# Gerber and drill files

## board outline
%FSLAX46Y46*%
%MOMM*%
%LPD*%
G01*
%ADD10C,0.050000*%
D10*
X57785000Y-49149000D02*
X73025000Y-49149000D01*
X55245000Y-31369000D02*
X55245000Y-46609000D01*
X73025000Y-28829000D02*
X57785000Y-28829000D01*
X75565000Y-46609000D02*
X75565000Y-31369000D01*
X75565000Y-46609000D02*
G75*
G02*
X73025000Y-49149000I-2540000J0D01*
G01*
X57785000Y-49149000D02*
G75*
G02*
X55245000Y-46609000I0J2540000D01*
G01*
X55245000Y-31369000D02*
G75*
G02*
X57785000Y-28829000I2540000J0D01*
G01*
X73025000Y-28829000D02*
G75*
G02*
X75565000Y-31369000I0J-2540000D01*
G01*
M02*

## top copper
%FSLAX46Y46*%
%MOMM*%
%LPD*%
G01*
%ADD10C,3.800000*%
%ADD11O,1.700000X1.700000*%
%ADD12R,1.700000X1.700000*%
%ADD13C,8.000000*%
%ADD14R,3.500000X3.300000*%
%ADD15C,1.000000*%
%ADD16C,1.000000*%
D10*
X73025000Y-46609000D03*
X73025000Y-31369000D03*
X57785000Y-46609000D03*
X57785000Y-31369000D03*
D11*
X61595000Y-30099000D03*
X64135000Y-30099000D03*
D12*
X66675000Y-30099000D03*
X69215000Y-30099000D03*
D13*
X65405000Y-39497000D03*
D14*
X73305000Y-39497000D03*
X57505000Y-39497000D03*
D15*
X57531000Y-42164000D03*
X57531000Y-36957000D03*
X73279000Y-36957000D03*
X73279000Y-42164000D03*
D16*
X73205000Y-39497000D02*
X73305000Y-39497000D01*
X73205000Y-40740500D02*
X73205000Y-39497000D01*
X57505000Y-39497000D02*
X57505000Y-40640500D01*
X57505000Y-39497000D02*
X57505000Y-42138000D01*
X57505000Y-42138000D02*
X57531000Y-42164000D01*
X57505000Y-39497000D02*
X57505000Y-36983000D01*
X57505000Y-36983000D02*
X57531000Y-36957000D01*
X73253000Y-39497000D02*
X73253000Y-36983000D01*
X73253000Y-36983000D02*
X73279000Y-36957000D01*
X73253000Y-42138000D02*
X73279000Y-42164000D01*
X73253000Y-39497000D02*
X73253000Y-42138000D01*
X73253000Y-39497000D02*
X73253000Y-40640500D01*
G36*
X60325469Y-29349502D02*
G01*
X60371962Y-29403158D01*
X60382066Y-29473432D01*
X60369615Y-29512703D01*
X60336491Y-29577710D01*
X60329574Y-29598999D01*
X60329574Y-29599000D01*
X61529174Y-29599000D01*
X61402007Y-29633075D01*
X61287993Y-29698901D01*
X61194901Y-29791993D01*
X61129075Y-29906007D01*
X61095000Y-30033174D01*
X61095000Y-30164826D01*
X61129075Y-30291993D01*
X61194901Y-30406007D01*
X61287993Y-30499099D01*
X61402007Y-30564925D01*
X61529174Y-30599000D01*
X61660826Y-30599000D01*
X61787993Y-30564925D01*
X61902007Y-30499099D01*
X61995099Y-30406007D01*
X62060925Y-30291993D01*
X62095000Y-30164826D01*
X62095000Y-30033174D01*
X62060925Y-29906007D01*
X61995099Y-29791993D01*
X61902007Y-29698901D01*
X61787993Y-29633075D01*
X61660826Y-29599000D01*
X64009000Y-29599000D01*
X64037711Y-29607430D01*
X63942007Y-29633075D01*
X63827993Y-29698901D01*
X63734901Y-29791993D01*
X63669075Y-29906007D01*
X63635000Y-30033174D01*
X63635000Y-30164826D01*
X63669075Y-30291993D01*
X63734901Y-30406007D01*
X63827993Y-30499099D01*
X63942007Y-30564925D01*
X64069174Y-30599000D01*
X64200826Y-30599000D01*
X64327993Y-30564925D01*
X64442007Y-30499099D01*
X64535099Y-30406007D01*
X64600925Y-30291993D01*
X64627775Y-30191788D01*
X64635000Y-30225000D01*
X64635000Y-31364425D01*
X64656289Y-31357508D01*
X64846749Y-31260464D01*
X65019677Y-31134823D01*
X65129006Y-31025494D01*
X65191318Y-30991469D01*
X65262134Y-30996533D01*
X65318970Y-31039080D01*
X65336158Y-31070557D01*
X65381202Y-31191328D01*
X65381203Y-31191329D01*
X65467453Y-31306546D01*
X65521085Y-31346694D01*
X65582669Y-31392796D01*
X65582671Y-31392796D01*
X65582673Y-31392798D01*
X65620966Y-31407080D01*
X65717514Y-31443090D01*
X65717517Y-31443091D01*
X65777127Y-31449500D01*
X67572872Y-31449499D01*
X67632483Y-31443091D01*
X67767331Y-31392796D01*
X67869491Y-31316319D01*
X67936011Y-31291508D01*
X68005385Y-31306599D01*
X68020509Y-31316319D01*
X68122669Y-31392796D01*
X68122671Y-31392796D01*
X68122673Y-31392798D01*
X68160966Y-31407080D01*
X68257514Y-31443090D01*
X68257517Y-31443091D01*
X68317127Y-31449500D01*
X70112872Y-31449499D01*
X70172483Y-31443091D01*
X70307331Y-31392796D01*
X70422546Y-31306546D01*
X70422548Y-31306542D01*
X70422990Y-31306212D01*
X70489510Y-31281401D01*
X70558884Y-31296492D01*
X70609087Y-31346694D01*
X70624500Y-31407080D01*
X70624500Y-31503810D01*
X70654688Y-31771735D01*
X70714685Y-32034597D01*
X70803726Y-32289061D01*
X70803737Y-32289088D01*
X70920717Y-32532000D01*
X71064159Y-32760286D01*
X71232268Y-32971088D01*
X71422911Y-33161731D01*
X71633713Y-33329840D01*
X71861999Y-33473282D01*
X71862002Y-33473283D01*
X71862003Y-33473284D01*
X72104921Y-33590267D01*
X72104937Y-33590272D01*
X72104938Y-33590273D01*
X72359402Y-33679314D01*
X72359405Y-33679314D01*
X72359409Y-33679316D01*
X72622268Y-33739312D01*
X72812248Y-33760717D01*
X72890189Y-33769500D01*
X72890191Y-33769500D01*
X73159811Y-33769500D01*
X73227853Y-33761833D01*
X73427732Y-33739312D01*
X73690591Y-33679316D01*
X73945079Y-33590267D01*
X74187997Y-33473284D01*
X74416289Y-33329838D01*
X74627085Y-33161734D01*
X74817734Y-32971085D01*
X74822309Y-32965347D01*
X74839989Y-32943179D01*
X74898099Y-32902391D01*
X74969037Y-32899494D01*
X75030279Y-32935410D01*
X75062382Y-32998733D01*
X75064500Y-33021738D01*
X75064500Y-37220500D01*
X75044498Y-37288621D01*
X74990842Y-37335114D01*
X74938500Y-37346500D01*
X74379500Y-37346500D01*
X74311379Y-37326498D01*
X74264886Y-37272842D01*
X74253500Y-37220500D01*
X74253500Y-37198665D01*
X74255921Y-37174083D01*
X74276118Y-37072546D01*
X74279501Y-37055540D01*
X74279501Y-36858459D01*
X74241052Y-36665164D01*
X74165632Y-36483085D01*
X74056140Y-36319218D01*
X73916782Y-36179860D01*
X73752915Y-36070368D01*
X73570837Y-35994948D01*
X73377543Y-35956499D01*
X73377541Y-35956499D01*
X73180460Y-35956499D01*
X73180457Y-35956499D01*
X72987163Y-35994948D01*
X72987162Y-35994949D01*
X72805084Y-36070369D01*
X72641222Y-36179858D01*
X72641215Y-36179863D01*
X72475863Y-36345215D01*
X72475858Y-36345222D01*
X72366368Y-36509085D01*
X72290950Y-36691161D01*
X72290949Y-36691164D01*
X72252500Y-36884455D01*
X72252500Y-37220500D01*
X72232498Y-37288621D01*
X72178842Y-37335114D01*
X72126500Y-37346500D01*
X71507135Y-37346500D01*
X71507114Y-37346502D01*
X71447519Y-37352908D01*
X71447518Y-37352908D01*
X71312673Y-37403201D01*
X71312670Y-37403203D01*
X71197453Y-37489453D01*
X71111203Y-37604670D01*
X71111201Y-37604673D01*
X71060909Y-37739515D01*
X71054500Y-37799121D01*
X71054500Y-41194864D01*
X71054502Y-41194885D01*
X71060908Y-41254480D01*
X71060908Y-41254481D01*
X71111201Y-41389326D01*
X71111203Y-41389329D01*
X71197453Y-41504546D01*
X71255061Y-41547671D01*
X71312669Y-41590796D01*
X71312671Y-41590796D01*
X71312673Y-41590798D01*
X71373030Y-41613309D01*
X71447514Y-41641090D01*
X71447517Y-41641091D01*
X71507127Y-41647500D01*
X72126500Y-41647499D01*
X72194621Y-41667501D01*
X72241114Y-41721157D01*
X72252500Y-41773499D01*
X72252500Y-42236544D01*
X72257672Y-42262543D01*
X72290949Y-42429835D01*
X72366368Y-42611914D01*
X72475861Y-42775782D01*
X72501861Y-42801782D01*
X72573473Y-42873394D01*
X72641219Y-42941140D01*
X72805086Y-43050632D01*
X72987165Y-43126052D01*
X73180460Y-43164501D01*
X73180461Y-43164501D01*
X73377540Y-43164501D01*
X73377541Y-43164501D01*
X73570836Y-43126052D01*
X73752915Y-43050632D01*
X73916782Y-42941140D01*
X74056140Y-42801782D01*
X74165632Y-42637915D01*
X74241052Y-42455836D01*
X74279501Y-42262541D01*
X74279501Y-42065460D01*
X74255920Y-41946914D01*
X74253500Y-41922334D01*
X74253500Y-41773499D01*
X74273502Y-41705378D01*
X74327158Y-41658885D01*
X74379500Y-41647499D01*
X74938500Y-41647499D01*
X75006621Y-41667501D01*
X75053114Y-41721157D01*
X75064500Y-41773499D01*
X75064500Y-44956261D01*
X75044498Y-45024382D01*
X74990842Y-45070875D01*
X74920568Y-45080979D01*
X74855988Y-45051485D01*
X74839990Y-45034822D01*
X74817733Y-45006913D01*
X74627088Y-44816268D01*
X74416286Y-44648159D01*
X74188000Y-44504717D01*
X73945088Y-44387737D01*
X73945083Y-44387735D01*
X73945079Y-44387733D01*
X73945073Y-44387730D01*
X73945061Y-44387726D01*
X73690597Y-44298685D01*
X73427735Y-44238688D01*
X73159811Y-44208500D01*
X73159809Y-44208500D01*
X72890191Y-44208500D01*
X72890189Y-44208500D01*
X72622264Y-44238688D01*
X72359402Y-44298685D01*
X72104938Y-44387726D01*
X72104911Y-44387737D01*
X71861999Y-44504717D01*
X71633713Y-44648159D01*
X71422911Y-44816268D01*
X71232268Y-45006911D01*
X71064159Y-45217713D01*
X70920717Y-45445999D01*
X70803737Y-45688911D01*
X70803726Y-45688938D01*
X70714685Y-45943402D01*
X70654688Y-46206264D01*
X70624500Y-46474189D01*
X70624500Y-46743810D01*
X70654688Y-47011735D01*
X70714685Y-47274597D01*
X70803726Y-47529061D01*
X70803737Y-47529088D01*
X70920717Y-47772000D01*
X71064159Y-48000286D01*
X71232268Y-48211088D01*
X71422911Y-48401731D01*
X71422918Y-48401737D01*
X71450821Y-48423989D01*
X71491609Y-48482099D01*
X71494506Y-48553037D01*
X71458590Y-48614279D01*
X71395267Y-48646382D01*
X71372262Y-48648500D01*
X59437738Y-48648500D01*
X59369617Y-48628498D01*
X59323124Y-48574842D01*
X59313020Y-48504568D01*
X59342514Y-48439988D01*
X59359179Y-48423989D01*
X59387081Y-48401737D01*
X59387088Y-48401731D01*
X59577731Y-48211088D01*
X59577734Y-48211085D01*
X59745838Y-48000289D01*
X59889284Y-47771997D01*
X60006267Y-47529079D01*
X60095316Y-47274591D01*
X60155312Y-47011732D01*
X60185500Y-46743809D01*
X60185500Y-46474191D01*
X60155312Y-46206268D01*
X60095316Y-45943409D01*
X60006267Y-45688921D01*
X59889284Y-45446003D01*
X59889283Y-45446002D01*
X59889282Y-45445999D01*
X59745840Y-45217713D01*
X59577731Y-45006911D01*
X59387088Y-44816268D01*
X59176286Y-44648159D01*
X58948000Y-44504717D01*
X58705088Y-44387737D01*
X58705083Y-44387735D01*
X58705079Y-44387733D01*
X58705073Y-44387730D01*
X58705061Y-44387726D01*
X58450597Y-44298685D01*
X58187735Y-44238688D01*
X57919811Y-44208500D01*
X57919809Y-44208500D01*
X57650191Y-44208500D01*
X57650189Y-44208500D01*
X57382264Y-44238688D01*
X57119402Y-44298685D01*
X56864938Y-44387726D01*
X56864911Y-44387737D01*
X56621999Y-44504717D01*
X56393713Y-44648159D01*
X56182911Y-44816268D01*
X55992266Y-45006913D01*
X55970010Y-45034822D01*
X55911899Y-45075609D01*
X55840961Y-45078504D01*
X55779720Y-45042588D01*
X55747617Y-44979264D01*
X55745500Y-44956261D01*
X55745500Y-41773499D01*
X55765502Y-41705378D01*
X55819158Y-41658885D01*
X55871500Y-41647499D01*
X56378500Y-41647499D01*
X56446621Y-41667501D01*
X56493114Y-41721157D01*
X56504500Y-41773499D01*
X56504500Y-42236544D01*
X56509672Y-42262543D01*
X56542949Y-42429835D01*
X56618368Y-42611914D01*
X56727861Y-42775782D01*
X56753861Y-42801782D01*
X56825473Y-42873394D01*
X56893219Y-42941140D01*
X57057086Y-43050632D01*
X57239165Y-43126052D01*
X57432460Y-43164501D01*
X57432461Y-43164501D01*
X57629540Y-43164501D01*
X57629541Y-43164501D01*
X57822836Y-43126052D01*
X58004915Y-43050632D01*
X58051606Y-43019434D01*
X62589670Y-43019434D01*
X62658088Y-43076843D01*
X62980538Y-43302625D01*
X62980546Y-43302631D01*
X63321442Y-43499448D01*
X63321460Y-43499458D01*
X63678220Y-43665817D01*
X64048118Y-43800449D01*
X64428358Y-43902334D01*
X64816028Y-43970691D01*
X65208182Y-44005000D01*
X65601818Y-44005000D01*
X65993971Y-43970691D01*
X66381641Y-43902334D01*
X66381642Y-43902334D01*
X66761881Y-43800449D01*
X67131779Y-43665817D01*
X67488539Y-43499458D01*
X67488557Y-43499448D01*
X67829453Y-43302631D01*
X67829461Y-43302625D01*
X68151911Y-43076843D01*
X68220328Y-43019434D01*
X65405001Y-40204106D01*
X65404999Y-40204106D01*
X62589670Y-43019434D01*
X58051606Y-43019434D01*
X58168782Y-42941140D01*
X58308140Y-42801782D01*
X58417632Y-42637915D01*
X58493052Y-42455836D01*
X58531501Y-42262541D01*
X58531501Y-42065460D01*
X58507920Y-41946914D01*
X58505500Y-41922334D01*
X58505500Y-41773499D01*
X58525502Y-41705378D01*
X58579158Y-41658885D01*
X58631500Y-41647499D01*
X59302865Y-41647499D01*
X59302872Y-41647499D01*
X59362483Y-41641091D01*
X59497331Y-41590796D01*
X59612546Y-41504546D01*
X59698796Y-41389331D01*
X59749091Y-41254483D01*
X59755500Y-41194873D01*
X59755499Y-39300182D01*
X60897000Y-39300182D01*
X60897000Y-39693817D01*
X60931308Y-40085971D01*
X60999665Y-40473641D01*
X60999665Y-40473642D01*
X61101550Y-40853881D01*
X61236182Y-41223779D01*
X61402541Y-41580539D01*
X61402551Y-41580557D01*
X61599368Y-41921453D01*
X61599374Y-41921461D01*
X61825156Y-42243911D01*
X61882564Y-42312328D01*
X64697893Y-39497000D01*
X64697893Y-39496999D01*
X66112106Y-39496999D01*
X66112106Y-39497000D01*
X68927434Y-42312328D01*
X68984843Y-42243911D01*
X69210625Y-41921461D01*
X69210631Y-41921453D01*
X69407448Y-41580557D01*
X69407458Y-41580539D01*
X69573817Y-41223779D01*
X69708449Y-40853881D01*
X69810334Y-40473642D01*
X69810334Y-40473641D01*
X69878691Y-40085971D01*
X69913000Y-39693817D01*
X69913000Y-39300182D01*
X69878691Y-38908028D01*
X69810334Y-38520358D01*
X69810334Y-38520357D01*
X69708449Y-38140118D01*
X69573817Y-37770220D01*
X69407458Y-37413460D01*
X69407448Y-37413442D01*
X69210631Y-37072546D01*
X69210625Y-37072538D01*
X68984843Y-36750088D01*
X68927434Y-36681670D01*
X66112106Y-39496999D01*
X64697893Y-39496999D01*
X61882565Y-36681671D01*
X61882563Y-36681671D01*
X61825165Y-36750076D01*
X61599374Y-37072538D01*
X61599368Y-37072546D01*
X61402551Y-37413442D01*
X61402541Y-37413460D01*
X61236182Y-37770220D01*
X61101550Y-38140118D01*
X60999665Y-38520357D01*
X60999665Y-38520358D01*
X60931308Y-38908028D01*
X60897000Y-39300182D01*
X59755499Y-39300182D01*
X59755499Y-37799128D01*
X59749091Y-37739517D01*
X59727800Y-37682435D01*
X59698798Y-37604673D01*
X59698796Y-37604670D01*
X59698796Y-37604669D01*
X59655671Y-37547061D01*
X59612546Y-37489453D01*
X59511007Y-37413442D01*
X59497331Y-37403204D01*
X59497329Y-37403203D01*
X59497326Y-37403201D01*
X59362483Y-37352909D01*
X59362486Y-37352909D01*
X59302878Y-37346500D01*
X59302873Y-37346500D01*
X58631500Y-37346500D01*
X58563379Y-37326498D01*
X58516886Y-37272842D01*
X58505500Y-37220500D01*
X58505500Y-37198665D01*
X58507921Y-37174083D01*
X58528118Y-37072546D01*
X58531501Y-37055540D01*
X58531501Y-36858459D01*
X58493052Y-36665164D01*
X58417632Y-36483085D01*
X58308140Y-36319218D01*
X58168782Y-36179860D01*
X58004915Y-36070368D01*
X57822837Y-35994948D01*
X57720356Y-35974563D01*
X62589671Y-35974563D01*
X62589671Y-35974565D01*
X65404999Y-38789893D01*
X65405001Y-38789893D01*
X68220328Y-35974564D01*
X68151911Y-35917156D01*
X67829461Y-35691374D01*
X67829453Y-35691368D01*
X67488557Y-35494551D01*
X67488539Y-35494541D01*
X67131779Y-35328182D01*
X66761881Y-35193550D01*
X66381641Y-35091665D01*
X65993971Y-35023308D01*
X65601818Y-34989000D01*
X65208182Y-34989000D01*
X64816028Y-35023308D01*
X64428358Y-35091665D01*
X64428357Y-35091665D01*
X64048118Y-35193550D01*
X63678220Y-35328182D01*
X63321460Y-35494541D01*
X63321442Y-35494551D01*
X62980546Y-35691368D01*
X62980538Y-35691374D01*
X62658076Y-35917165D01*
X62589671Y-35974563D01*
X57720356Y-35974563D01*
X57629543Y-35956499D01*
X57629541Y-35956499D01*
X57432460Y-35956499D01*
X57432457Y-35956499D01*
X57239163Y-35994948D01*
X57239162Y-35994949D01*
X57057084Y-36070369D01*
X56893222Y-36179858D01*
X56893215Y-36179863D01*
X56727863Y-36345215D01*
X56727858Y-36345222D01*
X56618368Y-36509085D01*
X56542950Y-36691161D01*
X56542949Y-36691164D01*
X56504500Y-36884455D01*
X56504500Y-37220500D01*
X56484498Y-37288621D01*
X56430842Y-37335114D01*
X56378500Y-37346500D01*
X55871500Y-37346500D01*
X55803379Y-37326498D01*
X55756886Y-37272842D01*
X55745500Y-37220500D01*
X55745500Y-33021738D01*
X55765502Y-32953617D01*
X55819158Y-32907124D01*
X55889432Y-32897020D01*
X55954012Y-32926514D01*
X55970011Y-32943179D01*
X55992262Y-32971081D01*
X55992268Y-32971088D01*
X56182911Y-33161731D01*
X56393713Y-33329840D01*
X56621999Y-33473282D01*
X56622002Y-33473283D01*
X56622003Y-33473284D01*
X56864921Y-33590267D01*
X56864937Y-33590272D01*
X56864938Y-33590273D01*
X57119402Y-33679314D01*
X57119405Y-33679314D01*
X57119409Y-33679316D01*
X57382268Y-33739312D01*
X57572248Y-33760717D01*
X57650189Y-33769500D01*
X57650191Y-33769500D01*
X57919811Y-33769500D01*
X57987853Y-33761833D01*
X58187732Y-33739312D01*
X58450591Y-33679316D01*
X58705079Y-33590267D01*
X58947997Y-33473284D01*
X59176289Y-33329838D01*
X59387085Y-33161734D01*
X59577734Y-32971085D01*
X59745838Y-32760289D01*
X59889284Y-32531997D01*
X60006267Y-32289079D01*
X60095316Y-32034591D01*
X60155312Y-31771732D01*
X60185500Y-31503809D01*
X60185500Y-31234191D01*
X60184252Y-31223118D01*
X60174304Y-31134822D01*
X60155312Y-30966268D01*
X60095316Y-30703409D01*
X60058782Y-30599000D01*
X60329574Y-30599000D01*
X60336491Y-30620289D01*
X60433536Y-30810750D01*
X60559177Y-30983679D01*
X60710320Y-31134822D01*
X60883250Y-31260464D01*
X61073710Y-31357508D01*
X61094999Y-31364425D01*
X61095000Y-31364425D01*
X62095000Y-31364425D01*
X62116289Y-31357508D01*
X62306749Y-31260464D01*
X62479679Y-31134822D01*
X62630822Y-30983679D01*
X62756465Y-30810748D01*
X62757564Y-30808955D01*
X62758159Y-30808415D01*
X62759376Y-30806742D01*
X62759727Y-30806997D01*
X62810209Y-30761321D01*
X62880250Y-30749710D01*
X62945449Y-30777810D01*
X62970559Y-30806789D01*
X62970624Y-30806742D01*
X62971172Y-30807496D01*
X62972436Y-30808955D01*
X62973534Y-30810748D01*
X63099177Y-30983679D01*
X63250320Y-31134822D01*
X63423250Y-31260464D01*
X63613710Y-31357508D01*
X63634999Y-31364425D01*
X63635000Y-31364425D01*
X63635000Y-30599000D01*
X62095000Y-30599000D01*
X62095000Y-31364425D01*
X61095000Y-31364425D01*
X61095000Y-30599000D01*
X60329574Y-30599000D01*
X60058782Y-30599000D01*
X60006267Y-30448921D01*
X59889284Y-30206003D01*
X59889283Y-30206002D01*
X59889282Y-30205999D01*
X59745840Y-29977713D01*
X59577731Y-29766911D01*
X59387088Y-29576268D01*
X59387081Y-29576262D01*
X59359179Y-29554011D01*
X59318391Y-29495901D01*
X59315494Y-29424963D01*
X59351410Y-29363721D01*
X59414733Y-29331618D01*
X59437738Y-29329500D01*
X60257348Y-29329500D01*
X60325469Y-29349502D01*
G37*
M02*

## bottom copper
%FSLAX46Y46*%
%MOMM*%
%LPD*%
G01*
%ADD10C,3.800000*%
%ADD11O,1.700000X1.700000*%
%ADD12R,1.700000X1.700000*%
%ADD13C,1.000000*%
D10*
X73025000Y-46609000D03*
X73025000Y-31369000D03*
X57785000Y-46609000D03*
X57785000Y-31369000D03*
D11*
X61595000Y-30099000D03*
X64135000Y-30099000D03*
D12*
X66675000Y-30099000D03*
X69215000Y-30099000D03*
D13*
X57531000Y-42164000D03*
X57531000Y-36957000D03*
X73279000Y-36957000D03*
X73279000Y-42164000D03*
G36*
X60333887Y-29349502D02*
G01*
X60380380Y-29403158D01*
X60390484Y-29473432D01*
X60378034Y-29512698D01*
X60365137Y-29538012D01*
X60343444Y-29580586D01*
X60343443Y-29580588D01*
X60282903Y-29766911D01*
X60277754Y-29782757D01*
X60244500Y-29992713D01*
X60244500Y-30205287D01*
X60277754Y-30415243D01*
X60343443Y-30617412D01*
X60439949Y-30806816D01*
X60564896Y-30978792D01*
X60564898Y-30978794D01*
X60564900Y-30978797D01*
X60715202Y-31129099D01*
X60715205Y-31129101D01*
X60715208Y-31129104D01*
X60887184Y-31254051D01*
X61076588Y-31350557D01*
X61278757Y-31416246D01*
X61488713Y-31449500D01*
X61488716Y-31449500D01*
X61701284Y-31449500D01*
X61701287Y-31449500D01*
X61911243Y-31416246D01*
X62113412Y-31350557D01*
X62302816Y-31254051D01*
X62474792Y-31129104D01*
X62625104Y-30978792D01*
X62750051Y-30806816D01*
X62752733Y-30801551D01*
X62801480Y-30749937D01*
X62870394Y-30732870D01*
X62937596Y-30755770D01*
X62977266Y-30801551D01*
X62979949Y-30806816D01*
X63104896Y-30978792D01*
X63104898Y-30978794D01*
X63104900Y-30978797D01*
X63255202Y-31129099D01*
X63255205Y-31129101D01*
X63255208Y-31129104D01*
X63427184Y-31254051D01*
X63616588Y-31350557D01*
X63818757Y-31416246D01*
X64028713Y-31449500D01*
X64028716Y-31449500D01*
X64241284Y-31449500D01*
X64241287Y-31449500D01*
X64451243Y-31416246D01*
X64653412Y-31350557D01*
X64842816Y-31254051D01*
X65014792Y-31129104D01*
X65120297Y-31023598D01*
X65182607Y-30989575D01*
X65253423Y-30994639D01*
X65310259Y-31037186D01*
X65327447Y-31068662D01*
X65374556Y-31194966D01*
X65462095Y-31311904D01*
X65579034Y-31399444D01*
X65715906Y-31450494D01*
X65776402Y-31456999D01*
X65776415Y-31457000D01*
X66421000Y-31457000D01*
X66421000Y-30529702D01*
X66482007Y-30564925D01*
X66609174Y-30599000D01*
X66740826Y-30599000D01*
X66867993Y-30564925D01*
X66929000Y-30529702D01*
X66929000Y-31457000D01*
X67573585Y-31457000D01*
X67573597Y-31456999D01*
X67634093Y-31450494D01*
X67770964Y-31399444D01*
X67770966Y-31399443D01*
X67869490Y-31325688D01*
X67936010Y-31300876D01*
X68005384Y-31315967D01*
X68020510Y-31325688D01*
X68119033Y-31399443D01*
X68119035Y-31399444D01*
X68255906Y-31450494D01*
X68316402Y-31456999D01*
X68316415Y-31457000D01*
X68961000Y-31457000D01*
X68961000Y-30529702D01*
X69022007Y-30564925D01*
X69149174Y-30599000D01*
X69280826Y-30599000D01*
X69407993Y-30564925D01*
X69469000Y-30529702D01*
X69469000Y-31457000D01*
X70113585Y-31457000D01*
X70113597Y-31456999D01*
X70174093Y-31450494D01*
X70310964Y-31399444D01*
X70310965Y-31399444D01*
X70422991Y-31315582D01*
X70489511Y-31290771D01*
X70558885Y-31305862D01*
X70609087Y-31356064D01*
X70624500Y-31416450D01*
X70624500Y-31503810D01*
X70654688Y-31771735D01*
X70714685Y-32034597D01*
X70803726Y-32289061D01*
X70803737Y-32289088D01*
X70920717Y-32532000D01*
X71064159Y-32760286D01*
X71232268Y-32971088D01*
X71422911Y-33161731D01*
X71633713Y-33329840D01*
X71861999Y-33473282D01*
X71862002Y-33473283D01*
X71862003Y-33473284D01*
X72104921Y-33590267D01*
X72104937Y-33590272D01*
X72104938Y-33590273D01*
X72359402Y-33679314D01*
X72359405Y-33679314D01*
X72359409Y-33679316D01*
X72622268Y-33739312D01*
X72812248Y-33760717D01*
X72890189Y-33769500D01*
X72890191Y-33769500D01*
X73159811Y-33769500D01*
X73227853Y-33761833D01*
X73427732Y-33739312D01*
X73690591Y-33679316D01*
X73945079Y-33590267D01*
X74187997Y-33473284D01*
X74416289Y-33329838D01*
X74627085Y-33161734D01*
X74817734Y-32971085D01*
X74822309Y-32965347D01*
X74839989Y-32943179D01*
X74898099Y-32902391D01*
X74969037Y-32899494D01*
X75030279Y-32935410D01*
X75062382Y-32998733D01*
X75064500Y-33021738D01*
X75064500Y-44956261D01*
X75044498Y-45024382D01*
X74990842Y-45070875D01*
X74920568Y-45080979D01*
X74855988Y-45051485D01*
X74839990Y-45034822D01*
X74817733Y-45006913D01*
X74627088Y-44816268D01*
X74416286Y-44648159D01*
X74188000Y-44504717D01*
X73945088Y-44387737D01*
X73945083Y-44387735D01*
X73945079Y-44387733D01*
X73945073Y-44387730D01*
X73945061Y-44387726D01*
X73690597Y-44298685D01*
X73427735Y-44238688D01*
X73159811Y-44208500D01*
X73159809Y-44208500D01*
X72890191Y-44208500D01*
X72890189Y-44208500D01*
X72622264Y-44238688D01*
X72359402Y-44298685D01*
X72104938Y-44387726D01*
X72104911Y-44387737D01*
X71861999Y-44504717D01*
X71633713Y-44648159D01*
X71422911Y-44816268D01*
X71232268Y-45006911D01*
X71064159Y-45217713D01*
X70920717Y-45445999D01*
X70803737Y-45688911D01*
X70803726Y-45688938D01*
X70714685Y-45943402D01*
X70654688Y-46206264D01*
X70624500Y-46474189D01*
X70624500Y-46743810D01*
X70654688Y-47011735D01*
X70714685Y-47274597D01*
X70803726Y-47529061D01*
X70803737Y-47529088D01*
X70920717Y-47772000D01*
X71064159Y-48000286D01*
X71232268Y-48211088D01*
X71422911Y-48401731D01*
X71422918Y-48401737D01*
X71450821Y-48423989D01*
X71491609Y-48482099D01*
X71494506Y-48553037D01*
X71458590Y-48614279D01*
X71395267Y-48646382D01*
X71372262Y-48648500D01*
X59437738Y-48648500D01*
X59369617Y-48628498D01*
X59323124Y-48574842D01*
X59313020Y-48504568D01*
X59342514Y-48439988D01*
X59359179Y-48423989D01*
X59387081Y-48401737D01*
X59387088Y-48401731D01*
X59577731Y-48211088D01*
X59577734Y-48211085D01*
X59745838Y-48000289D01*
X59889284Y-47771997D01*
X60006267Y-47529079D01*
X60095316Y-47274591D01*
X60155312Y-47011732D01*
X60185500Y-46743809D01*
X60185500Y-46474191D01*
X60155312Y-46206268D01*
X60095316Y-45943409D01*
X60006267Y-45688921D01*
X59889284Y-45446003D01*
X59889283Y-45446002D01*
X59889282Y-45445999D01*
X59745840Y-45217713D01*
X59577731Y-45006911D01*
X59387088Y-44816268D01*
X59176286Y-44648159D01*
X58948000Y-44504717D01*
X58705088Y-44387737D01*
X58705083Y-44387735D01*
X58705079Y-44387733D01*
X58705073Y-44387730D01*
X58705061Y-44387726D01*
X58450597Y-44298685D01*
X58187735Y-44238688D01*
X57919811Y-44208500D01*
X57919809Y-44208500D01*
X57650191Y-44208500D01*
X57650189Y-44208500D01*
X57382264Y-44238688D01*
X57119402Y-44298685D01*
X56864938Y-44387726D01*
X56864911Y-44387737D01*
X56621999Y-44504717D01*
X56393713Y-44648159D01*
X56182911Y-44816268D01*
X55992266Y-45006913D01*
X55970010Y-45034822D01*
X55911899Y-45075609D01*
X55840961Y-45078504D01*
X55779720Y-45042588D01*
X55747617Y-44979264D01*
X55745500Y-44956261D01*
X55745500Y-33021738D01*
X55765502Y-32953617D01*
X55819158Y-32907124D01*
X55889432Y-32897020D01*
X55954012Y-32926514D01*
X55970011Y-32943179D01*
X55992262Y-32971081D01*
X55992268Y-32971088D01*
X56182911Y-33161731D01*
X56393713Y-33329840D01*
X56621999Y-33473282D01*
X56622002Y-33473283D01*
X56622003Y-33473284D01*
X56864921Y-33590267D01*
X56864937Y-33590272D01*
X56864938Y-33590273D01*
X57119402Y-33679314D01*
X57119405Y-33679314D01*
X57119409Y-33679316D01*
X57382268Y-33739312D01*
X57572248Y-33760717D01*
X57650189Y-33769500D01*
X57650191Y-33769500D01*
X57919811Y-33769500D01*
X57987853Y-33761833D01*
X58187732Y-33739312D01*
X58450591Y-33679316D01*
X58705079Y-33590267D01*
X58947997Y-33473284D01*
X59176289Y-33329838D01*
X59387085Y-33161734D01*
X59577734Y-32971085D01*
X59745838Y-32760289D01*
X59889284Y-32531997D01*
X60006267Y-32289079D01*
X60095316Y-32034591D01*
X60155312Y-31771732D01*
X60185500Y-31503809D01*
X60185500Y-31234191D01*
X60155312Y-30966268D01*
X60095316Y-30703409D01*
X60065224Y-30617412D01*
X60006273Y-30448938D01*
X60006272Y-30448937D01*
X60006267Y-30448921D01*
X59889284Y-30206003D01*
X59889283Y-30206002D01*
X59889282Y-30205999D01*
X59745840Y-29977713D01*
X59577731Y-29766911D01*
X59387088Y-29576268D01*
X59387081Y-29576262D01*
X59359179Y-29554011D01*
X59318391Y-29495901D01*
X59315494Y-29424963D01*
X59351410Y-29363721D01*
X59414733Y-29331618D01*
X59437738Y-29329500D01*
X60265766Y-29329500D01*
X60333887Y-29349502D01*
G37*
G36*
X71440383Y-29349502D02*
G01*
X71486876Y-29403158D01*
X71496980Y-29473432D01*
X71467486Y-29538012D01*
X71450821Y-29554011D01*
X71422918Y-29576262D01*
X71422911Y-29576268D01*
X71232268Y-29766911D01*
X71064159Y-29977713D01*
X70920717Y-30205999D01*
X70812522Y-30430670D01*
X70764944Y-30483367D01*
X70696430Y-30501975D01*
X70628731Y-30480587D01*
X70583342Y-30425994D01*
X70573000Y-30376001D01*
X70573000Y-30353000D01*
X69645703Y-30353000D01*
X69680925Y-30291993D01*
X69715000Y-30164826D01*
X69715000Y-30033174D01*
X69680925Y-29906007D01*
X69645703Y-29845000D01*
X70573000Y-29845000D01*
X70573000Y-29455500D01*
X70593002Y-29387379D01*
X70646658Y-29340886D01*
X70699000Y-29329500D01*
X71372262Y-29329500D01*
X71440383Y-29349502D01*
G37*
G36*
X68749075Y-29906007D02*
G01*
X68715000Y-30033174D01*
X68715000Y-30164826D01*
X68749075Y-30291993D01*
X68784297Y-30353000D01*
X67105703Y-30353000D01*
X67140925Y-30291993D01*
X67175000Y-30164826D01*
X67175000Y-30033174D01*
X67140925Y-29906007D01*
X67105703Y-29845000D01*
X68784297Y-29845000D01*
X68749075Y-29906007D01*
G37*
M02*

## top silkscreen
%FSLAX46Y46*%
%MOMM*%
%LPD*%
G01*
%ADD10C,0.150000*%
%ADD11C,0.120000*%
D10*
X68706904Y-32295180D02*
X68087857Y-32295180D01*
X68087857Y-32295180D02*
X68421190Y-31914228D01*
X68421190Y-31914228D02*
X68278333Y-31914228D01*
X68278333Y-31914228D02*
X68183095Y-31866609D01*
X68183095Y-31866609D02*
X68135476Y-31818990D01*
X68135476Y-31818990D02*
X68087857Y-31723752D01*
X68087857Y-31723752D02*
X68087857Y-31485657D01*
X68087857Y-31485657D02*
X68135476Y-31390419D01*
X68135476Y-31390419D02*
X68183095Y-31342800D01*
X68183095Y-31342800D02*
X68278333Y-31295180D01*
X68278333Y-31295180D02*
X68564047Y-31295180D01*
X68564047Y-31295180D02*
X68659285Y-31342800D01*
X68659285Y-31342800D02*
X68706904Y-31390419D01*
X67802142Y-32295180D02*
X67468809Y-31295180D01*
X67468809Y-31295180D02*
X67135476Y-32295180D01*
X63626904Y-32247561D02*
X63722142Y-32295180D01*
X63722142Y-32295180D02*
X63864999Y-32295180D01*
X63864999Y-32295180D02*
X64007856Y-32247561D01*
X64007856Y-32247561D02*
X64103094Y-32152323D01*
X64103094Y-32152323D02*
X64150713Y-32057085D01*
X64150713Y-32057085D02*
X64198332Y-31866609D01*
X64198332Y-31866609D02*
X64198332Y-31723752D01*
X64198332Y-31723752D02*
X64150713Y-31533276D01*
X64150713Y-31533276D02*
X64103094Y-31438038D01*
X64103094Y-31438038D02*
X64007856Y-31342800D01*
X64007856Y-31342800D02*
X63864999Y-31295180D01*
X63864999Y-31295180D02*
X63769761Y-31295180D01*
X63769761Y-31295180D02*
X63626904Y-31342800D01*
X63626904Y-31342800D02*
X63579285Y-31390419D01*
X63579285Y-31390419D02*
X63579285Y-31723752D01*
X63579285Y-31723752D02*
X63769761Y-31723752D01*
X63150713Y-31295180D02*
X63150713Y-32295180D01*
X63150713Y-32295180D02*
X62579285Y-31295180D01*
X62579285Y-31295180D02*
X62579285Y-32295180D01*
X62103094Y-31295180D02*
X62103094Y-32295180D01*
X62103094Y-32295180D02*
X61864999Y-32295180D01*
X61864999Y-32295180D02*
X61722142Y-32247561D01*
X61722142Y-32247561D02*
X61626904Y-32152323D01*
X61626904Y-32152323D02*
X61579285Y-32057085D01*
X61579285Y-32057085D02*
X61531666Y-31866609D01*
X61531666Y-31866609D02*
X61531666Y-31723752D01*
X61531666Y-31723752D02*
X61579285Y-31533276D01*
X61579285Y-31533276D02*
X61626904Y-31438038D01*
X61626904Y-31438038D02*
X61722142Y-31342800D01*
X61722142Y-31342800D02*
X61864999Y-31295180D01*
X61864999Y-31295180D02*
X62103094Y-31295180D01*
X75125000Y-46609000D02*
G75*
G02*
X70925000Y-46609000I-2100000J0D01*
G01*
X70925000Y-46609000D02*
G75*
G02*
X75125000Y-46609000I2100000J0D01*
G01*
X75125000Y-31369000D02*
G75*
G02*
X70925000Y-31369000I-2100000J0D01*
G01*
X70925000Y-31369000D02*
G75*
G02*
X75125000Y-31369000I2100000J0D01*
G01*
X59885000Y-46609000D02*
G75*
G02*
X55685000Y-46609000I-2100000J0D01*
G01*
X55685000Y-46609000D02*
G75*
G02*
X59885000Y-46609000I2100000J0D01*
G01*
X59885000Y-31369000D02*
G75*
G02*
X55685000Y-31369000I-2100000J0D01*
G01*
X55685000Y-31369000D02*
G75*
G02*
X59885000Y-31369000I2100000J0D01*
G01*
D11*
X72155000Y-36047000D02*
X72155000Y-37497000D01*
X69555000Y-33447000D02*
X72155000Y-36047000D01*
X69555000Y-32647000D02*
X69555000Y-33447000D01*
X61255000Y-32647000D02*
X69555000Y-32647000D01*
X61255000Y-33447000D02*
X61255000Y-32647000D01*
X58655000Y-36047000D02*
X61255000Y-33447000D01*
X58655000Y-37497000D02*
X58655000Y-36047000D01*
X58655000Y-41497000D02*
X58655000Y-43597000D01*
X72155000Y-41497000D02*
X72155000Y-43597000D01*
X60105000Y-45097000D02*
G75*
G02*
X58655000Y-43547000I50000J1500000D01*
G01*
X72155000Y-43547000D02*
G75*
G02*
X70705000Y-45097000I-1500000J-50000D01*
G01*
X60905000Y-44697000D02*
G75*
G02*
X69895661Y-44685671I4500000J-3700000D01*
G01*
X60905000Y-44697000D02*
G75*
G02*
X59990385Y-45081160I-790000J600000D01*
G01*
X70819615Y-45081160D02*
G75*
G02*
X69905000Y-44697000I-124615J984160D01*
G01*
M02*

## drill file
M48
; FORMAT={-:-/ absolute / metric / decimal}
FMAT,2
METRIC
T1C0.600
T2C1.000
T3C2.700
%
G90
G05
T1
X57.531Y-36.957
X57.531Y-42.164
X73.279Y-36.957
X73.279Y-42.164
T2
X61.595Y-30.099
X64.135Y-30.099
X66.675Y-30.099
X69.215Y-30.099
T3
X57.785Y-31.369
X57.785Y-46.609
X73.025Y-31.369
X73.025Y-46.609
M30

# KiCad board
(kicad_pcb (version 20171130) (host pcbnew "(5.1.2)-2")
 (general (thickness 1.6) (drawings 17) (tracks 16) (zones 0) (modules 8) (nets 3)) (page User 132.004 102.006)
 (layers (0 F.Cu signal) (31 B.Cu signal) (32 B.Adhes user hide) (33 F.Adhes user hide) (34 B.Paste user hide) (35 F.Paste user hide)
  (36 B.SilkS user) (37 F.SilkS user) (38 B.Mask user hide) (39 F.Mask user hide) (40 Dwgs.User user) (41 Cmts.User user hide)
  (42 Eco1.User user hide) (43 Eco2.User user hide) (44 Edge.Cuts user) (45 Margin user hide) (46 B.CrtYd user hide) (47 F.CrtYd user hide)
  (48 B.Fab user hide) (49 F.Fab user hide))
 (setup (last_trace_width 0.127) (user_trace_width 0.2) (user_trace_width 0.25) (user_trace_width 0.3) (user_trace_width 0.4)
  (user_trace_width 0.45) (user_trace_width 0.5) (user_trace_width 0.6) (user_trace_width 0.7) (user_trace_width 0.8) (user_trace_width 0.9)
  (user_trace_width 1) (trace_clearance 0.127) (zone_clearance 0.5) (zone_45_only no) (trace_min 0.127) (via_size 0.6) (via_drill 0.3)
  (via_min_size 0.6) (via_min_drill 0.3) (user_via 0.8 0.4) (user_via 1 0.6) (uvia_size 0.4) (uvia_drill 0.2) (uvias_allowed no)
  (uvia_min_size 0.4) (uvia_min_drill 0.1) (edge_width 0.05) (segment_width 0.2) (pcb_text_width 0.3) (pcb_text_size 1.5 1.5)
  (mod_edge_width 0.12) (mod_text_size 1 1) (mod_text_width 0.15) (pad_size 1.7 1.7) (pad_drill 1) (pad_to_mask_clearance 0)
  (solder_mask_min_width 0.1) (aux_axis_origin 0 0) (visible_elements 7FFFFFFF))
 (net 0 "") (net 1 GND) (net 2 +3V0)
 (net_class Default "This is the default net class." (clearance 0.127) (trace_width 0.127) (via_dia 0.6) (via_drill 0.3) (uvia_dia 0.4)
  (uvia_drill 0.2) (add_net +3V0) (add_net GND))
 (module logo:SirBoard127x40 (layer B.Cu) (at 65.405 38.735)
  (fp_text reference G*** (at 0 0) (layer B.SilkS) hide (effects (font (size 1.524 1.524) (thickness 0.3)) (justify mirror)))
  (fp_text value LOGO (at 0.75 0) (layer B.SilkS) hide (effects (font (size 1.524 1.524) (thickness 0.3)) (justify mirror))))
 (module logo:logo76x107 (layer B.Cu) (at 65.405 44.8945)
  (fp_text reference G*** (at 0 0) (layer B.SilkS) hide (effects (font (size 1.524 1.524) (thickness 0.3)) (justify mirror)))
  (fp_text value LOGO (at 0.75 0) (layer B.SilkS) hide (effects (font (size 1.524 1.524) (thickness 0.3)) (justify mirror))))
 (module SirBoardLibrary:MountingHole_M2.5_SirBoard (layer F.Cu) (at 73.025 46.609)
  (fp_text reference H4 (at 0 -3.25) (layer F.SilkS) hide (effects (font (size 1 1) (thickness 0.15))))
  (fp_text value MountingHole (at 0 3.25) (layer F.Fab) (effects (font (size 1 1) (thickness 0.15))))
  (fp_circle (center 0 0) (end 2.1 0) (layer F.SilkS) (width 0.15))
  (pad 1 thru_hole circle (at 0 0) (size 3.8 3.8) (drill 2.7) (layers *.Cu *.Mask)))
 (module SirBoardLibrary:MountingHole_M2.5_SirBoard (layer F.Cu) (at 73.025 31.369)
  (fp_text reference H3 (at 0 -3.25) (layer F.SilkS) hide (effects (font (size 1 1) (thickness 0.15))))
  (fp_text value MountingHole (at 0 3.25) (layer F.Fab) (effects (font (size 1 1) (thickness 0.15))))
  (fp_circle (center 0 0) (end 2.1 0) (layer F.SilkS) (width 0.15))
  (pad 1 thru_hole circle (at 0 0) (size 3.8 3.8) (drill 2.7) (layers *.Cu *.Mask)))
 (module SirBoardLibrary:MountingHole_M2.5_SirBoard (layer F.Cu) (at 57.785 46.609)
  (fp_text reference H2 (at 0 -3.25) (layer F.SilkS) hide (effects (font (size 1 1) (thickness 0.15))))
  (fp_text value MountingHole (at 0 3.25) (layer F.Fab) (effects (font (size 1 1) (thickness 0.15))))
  (fp_circle (center 0 0) (end 2.1 0) (layer F.SilkS) (width 0.15))
  (pad 1 thru_hole circle (at 0 0) (size 3.8 3.8) (drill 2.7) (layers *.Cu *.Mask)))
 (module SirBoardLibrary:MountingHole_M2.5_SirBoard (layer F.Cu) (at 57.785 31.369)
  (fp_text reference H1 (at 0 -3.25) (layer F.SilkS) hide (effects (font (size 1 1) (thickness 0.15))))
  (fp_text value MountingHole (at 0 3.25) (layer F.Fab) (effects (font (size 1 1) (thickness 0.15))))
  (fp_circle (center 0 0) (end 2.1 0) (layer F.SilkS) (width 0.15))
  (pad 1 thru_hole circle (at 0 0) (size 3.8 3.8) (drill 2.7) (layers *.Cu *.Mask)))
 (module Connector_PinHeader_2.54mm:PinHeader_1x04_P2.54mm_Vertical (layer F.Cu) (at 69.215 30.099 270)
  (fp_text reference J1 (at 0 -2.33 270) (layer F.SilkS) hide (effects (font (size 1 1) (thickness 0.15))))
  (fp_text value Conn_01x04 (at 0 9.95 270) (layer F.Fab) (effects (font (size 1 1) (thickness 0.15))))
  (pad 4 thru_hole oval (at 0 7.62 270) (size 1.7 1.7) (drill 1) (layers *.Cu *.Mask) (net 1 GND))
  (pad 3 thru_hole oval (at 0 5.08 270) (size 1.7 1.7) (drill 1) (layers *.Cu *.Mask) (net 1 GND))
  (pad 2 thru_hole rect (at 0 2.54 270) (size 1.7 1.7) (drill 1) (layers *.Cu *.Mask) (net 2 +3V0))
  (pad 1 thru_hole rect (at 0 0 270) (size 1.7 1.7) (drill 1) (layers *.Cu *.Mask) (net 2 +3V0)))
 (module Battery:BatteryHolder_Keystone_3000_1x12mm (layer F.Cu) (at 65.405 39.497)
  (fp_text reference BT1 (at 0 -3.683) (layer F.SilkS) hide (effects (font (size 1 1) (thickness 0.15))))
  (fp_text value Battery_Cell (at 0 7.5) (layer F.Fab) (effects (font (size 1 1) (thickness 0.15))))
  (fp_line (start 6.75 -3.45) (end 6.75 -2) (layer F.SilkS) (width 0.12))
  (fp_line (start 4.15 -6.05) (end 6.75 -3.45) (layer F.SilkS) (width 0.12))
  (fp_line (start 4.15 -6.85) (end 4.15 -6.05) (layer F.SilkS) (width 0.12))
  (fp_line (start -4.15 -6.85) (end 4.15 -6.85) (layer F.SilkS) (width 0.12))
  (fp_line (start -4.15 -6.05) (end -4.15 -6.85) (layer F.SilkS) (width 0.12))
  (fp_line (start -6.75 -3.45) (end -4.15 -6.05) (layer F.SilkS) (width 0.12))
  (fp_line (start -6.75 -2) (end -6.75 -3.45) (layer F.SilkS) (width 0.12))
  (fp_line (start -6.75 2) (end -6.75 4.1) (layer F.SilkS) (width 0.12))
  (fp_line (start 6.75 2) (end 6.75 4.1) (layer F.SilkS) (width 0.12))
  (fp_arc (start -5.25 4.1) (end -5.3 5.6) (angle 90) (layer F.SilkS) (width 0.12))
  (fp_arc (start 5.25 4.1) (end 5.3 5.6) (angle -90) (layer F.SilkS) (width 0.12))
  (fp_arc (start 0 8.9) (end -4.5 5.2) (angle 101) (layer F.SilkS) (width 0.12))
  (fp_arc (start -5.29 4.6) (end -4.5 5.2) (angle 60) (layer F.SilkS) (width 0.12))
  (fp_arc (start 5.29 4.6) (end 4.5 5.2) (angle -60) (layer F.SilkS) (width 0.12))
  (pad 2 smd circle (at 0 0) (size 8 8) (layers F.Cu F.Mask) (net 1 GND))
  (pad 1 smd rect (at 7.9 0) (size 3.5 3.3) (layers F.Cu F.Paste F.Mask) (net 2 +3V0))
  (pad 1 smd rect (at -7.9 0) (size 3.5 3.3) (layers F.Cu F.Paste F.Mask) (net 2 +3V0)))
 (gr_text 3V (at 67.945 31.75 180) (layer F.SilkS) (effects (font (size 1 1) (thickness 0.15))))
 (gr_line (start 57.785 49.149) (end 73.025 49.149) (layer Edge.Cuts) (width 0.05))
 (gr_line (start 55.245 31.369) (end 55.245 46.609) (layer Edge.Cuts) (width 0.05))
 (gr_line (start 73.025 28.829) (end 57.785 28.829) (layer Edge.Cuts) (width 0.05))
 (gr_line (start 75.565 46.609) (end 75.565 31.369) (layer Edge.Cuts) (width 0.05))
 (gr_arc (start 73.025 46.609) (end 73.025 49.149) (angle -90) (layer Edge.Cuts) (width 0.05))
 (gr_arc (start 57.785 46.609) (end 55.245 46.609) (angle -90) (layer Edge.Cuts) (width 0.05))
 (gr_arc (start 57.785 31.369) (end 57.785 28.829) (angle -90) (layer Edge.Cuts) (width 0.05))
 (gr_arc (start 73.025 31.369) (end 75.565 31.369) (angle -90) (layer Edge.Cuts) (width 0.05))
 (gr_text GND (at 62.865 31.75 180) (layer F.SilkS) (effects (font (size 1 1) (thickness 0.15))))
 (segment (start 73.205 39.497) (end 73.305 39.497) (width 1) (layer F.Cu) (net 2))
 (segment (start 73.205 40.7405) (end 73.205 39.497) (width 1) (layer F.Cu) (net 2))
 (segment (start 57.505 39.497) (end 57.505 40.6405) (width 1) (layer F.Cu) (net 2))
 (via (at 57.531 42.164) (size 1) (drill 0.6) (layers F.Cu B.Cu) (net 2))
 (segment (start 57.505 39.497) (end 57.505 42.138) (width 1) (layer F.Cu) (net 2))
 (segment (start 57.505 42.138) (end 57.531 42.164) (width 1) (layer F.Cu) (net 2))
 (via (at 57.531 36.957) (size 1) (drill 0.6) (layers F.Cu B.Cu) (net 2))
 (segment (start 57.505 39.497) (end 57.505 36.983) (width 1) (layer F.Cu) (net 2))
 (segment (start 57.505 36.983) (end 57.531 36.957) (width 1) (layer F.Cu) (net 2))
 (segment (start 73.253 39.497) (end 73.253 36.983) (width 1) (layer F.Cu) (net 2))
 (segment (start 73.253 36.983) (end 73.279 36.957) (width 1) (layer F.Cu) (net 2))
 (segment (start 73.253 42.138) (end 73.279 42.164) (width 1) (layer F.Cu) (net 2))
 (segment (start 73.253 39.497) (end 73.253 42.138) (width 1) (layer F.Cu) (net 2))
 (via (at 73.279 36.957) (size 1) (drill 0.6) (layers F.Cu B.Cu) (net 2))
 (via (at 73.279 42.164) (size 1) (drill 0.6) (layers F.Cu B.Cu) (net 2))
 (segment (start 73.253 39.497) (end 73.253 40.6405) (width 1) (layer F.Cu) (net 2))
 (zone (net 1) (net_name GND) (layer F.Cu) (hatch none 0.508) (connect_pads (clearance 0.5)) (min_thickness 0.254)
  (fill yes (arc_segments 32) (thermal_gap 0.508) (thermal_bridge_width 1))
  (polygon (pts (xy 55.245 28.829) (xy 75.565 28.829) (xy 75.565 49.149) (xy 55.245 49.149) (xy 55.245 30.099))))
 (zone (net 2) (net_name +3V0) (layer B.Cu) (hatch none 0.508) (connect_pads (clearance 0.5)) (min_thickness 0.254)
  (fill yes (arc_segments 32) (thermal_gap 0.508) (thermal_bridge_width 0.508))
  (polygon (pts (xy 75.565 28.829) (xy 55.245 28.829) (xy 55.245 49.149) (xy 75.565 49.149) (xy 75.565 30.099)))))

